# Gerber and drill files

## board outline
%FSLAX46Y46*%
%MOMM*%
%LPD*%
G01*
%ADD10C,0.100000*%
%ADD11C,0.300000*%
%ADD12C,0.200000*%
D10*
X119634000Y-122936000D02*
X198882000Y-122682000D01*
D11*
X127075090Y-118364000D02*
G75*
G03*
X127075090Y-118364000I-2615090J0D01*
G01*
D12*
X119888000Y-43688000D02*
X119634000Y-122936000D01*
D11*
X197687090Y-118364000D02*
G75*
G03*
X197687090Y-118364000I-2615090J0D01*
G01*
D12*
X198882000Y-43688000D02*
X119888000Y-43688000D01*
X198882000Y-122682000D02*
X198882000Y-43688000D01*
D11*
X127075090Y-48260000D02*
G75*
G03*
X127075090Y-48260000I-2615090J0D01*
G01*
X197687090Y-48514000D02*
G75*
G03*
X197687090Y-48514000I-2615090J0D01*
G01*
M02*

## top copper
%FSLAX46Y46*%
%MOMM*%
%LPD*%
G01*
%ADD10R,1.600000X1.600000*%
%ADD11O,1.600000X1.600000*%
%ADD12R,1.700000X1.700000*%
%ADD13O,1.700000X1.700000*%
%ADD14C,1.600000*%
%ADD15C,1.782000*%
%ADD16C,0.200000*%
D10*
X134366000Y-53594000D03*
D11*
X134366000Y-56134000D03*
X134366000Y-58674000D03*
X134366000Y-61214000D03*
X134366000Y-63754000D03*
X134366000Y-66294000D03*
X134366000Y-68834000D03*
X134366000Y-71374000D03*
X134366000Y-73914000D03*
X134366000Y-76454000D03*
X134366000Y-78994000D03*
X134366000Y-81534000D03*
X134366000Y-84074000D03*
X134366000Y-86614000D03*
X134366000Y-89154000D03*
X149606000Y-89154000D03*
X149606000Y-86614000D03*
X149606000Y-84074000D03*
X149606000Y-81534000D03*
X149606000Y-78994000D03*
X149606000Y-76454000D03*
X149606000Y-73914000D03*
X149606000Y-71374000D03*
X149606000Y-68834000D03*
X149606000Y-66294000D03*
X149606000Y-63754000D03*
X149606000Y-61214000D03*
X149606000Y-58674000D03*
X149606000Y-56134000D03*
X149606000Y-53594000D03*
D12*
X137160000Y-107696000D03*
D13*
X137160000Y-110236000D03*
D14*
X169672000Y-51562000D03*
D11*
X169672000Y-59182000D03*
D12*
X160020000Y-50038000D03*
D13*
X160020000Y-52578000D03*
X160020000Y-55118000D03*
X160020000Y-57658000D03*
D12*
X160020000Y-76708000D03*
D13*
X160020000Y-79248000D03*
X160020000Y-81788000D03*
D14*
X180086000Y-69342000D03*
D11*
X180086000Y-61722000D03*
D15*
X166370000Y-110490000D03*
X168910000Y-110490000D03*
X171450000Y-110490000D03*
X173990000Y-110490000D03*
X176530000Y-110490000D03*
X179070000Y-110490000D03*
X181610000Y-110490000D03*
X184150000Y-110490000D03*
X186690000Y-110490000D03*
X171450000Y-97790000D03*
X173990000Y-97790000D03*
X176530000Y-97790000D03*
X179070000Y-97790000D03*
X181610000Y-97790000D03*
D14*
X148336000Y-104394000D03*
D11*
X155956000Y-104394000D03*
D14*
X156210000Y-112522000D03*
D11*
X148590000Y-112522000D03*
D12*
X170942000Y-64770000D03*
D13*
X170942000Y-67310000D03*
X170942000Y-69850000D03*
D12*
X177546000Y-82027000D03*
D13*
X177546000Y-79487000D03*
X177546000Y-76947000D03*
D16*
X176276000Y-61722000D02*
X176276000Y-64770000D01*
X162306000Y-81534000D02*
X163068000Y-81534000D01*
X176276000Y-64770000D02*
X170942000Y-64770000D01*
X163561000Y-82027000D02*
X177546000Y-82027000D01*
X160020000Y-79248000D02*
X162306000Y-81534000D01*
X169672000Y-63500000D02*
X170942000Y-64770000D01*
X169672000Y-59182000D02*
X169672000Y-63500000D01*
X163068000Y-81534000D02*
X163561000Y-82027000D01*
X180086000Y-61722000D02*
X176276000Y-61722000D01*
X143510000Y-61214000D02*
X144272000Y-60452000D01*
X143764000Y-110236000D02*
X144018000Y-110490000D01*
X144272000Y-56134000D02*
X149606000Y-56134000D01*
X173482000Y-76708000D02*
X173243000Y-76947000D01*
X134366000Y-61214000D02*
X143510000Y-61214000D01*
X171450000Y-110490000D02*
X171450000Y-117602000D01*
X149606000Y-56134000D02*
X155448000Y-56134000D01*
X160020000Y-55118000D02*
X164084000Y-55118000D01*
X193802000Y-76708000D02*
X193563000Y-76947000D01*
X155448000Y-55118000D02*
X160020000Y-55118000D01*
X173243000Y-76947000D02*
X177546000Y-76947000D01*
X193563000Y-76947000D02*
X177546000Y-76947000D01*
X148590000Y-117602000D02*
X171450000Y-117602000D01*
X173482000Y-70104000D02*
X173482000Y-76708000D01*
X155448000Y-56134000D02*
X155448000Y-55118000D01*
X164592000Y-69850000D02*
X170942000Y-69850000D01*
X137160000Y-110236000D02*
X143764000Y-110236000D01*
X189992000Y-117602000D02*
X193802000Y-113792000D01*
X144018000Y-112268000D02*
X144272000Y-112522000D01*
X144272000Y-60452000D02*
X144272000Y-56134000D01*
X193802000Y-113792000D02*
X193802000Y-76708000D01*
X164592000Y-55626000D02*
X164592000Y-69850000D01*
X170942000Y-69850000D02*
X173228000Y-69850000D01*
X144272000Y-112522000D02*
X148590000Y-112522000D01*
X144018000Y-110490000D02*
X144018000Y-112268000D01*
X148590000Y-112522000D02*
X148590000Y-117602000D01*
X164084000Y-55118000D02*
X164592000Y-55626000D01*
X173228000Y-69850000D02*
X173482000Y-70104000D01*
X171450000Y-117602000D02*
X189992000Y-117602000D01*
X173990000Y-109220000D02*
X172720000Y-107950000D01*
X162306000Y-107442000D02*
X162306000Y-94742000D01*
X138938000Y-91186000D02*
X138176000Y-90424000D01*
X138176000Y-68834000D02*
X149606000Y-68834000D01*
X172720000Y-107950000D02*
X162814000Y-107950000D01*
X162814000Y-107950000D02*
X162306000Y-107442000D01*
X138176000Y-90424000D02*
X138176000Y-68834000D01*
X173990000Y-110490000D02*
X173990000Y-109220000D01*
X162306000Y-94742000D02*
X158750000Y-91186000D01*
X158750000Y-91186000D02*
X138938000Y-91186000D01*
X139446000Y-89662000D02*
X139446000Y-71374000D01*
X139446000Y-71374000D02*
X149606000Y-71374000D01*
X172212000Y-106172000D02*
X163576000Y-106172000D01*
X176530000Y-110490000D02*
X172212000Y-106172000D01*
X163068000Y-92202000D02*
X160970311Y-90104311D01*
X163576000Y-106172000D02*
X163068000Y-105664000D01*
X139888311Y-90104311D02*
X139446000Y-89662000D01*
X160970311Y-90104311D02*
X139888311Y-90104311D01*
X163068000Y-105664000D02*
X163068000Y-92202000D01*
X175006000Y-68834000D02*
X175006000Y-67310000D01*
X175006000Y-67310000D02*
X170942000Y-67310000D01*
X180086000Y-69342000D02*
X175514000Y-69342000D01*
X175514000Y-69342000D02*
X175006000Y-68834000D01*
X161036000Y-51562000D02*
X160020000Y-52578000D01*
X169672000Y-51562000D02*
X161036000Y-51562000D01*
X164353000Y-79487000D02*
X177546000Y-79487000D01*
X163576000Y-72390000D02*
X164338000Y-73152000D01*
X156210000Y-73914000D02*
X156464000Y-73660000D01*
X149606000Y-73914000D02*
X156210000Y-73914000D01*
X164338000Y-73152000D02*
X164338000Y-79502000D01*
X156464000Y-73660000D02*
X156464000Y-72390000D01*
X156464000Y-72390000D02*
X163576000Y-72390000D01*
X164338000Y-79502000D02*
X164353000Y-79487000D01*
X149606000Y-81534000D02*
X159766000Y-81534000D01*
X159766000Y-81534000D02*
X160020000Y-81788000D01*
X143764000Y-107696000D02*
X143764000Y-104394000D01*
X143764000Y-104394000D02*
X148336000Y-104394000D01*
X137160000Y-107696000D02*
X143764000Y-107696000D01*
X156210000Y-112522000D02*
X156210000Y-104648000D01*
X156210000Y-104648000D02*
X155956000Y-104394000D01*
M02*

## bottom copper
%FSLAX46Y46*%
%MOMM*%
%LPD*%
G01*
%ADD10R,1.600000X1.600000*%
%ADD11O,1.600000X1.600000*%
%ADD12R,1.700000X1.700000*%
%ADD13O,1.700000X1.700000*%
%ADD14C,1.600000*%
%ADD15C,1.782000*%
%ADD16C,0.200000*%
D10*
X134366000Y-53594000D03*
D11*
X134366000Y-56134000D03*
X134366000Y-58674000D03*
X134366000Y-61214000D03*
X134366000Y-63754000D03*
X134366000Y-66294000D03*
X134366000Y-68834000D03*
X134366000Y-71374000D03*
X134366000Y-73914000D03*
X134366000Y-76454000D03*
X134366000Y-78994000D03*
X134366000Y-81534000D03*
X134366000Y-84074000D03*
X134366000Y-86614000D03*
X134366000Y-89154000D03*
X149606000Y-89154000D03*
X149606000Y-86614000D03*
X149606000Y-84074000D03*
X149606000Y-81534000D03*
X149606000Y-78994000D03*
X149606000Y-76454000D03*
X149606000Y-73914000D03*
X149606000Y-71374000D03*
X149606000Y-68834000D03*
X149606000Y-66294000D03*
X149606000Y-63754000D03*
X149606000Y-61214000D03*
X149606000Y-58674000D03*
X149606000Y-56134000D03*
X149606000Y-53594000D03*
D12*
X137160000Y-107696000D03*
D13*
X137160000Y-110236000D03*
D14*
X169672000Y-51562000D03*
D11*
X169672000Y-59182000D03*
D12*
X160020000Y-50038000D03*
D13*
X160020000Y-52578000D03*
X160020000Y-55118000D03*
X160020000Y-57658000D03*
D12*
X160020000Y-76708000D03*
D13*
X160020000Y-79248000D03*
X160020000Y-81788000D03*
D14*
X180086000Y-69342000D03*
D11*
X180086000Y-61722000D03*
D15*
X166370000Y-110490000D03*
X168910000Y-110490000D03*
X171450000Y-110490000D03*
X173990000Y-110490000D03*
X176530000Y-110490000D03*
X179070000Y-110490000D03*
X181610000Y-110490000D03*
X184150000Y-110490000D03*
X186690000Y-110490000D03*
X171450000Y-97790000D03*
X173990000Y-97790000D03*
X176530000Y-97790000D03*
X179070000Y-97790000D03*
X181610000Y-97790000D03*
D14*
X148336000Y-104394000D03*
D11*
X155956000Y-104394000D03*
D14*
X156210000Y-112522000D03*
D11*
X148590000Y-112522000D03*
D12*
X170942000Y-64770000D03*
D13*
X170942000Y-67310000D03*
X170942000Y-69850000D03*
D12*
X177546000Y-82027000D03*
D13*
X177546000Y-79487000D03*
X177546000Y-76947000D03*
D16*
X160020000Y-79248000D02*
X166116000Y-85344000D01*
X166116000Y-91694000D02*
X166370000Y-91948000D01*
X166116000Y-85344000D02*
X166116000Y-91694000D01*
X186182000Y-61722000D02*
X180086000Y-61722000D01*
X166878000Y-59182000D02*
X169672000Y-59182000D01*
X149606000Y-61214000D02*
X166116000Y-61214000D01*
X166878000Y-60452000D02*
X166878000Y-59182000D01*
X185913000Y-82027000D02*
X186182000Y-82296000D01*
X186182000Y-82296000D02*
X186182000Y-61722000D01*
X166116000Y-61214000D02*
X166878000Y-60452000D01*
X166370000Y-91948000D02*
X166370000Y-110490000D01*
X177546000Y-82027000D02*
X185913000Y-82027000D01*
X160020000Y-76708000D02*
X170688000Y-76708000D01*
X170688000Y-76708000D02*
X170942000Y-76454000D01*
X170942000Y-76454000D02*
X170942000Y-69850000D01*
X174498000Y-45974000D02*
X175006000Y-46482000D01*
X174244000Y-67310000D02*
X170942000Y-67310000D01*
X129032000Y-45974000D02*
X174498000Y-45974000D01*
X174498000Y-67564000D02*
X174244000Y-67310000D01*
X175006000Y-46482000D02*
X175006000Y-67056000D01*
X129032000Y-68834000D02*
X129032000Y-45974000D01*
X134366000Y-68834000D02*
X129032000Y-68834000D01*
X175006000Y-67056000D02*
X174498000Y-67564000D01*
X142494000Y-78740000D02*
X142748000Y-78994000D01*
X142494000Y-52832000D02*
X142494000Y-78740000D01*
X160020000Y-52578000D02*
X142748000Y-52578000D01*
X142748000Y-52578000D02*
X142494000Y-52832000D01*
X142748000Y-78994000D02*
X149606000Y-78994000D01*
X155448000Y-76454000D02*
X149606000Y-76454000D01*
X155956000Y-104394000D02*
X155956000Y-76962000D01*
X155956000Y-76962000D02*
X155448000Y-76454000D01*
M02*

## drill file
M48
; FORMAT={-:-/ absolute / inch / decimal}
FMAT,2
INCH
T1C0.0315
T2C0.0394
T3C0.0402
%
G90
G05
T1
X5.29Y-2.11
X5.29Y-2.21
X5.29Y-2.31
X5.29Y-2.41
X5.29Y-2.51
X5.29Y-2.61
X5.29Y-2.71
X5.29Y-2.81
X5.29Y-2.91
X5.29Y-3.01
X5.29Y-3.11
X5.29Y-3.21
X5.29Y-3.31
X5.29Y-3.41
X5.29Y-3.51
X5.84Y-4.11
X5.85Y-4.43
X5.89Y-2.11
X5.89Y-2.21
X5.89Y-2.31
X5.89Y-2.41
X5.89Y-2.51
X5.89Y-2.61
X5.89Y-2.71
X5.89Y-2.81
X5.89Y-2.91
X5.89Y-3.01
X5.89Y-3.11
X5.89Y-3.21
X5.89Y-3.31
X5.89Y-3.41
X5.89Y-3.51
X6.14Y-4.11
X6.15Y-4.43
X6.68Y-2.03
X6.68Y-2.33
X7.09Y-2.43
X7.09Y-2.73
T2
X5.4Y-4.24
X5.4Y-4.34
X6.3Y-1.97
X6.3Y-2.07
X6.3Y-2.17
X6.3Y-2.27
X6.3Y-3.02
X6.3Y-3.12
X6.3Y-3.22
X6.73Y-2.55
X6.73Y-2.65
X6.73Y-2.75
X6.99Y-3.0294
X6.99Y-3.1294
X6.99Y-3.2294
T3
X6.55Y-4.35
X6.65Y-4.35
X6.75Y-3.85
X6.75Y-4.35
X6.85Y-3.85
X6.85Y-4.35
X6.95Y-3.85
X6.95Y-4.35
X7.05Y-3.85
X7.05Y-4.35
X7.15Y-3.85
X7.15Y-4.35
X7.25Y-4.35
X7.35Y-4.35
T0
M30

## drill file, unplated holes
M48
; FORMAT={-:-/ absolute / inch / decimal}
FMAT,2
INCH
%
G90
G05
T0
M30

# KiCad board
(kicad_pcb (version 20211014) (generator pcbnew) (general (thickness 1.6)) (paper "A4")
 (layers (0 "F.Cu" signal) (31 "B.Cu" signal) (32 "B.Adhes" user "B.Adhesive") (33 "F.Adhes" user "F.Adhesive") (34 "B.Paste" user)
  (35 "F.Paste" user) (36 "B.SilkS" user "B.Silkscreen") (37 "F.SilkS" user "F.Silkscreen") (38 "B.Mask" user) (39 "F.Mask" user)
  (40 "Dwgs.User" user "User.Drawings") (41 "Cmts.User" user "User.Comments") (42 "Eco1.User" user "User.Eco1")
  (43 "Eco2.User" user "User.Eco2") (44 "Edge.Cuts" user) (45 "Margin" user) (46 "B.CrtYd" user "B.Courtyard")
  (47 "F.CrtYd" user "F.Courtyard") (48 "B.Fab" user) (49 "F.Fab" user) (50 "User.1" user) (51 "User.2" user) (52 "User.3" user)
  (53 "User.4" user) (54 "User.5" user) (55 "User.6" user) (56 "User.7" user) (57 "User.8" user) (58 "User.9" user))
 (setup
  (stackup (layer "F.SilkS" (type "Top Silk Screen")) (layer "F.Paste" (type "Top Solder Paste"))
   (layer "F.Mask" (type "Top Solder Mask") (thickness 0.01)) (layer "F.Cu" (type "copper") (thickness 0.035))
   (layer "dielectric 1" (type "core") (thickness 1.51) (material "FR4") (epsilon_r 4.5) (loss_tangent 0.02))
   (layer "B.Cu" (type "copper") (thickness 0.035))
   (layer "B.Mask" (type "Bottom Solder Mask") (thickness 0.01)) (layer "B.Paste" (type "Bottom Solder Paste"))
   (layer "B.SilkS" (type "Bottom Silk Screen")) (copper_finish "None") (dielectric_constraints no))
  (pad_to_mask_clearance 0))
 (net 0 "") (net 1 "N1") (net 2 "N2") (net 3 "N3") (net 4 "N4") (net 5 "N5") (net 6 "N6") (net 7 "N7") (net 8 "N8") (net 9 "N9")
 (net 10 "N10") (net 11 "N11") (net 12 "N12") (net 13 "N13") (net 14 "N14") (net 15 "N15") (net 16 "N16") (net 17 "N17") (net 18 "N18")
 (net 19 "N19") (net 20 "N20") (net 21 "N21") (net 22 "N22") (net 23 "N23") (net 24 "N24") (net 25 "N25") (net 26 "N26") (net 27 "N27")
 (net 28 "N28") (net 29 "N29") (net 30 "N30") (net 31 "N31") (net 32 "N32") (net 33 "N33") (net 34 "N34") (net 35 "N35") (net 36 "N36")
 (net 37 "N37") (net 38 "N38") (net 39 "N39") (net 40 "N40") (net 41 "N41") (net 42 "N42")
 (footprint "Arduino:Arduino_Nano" (layer "F.Cu") (at 134.366 53.594)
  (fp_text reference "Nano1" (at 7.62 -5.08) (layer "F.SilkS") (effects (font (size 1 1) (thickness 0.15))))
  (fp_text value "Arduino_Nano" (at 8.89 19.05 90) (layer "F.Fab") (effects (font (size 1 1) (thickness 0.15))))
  (pad "1" thru_hole rect locked (at 0 0) (size 1.6 1.6) (drill 0.8) (layers *.Cu *.Mask) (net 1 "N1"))
  (pad "2" thru_hole oval locked (at 0 2.54) (size 1.6 1.6) (drill 0.8) (layers *.Cu *.Mask) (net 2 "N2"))
  (pad "3" thru_hole oval locked (at 0 5.08) (size 1.6 1.6) (drill 0.8) (layers *.Cu *.Mask) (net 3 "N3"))
  (pad "4" thru_hole oval locked (at 0 7.62) (size 1.6 1.6) (drill 0.8) (layers *.Cu *.Mask) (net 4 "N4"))
  (pad "5" thru_hole oval locked (at 0 10.16) (size 1.6 1.6) (drill 0.8) (layers *.Cu *.Mask) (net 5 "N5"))
  (pad "6" thru_hole oval locked (at 0 12.7) (size 1.6 1.6) (drill 0.8) (layers *.Cu *.Mask) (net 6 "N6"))
  (pad "7" thru_hole oval locked (at 0 15.24) (size 1.6 1.6) (drill 0.8) (layers *.Cu *.Mask) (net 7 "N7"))
  (pad "8" thru_hole oval locked (at 0 17.78) (size 1.6 1.6) (drill 0.8) (layers *.Cu *.Mask) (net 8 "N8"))
  (pad "9" thru_hole oval locked (at 0 20.32) (size 1.6 1.6) (drill 0.8) (layers *.Cu *.Mask) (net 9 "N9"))
  (pad "10" thru_hole oval locked (at 0 22.86) (size 1.6 1.6) (drill 0.8) (layers *.Cu *.Mask) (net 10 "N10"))
  (pad "11" thru_hole oval locked (at 0 25.4) (size 1.6 1.6) (drill 0.8) (layers *.Cu *.Mask) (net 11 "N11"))
  (pad "12" thru_hole oval locked (at 0 27.94) (size 1.6 1.6) (drill 0.8) (layers *.Cu *.Mask) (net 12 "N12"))
  (pad "13" thru_hole oval locked (at 0 30.48) (size 1.6 1.6) (drill 0.8) (layers *.Cu *.Mask) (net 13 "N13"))
  (pad "14" thru_hole oval locked (at 0 33.02) (size 1.6 1.6) (drill 0.8) (layers *.Cu *.Mask) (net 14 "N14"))
  (pad "15" thru_hole oval locked (at 0 35.56) (size 1.6 1.6) (drill 0.8) (layers *.Cu *.Mask) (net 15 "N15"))
  (pad "16" thru_hole oval locked (at 15.24 35.56) (size 1.6 1.6) (drill 0.8) (layers *.Cu *.Mask) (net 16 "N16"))
  (pad "17" thru_hole oval locked (at 15.24 33.02) (size 1.6 1.6) (drill 0.8) (layers *.Cu *.Mask) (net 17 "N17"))
  (pad "18" thru_hole oval locked (at 15.24 30.48) (size 1.6 1.6) (drill 0.8) (layers *.Cu *.Mask) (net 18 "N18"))
  (pad "19" thru_hole oval locked (at 15.24 27.94) (size 1.6 1.6) (drill 0.8) (layers *.Cu *.Mask) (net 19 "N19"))
  (pad "20" thru_hole oval locked (at 15.24 25.4) (size 1.6 1.6) (drill 0.8) (layers *.Cu *.Mask) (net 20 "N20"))
  (pad "21" thru_hole oval locked (at 15.24 22.86) (size 1.6 1.6) (drill 0.8) (layers *.Cu *.Mask) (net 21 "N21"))
  (pad "22" thru_hole oval locked (at 15.24 20.32) (size 1.6 1.6) (drill 0.8) (layers *.Cu *.Mask) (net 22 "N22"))
  (pad "23" thru_hole oval locked (at 15.24 17.78) (size 1.6 1.6) (drill 0.8) (layers *.Cu *.Mask) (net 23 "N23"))
  (pad "24" thru_hole oval locked (at 15.24 15.24) (size 1.6 1.6) (drill 0.8) (layers *.Cu *.Mask) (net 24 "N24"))
  (pad "25" thru_hole oval locked (at 15.24 12.7) (size 1.6 1.6) (drill 0.8) (layers *.Cu *.Mask) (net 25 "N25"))
  (pad "26" thru_hole oval locked (at 15.24 10.16) (size 1.6 1.6) (drill 0.8) (layers *.Cu *.Mask) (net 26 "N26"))
  (pad "27" thru_hole oval locked (at 15.24 7.62) (size 1.6 1.6) (drill 0.8) (layers *.Cu *.Mask) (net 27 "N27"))
  (pad "28" thru_hole oval locked (at 15.24 5.08) (size 1.6 1.6) (drill 0.8) (layers *.Cu *.Mask) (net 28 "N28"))
  (pad "29" thru_hole oval locked (at 15.24 2.54) (size 1.6 1.6) (drill 0.8) (layers *.Cu *.Mask) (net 4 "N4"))
  (pad "30" thru_hole oval locked (at 15.24 0) (size 1.6 1.6) (drill 0.8) (layers *.Cu *.Mask) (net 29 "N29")))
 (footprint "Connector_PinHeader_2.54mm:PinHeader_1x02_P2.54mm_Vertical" (layer "F.Cu") (at 137.16 107.696)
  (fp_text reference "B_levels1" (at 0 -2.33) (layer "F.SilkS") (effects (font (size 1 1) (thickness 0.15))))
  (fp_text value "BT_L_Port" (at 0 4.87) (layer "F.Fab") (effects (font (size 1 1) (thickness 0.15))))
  (pad "1" thru_hole rect (at 0 0) (size 1.7 1.7) (drill 1) (layers *.Cu *.Mask) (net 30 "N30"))
  (pad "2" thru_hole oval (at 0 2.54) (size 1.7 1.7) (drill 1) (layers *.Cu *.Mask) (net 4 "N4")))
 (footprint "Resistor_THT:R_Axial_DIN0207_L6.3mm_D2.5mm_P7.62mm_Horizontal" (layer "F.Cu") (at 169.672 51.562 -90)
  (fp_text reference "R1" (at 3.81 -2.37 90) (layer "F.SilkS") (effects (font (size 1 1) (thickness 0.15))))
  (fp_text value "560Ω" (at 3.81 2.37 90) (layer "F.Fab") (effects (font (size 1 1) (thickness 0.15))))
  (pad "1" thru_hole circle (at 0 0 270) (size 1.6 1.6) (drill 0.8) (layers *.Cu *.Mask) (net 20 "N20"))
  (pad "2" thru_hole oval (at 7.62 0 270) (size 1.6 1.6) (drill 0.8) (layers *.Cu *.Mask) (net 27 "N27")))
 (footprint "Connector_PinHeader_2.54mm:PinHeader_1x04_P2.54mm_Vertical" (layer "F.Cu") (at 160.02 50.038)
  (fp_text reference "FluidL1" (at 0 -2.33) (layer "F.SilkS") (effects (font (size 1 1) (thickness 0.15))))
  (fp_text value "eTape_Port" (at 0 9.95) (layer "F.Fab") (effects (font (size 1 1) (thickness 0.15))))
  (pad "1" thru_hole rect (at 0 0) (size 1.7 1.7) (drill 1) (layers *.Cu *.Mask) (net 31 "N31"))
  (pad "2" thru_hole oval (at 0 2.54) (size 1.7 1.7) (drill 1) (layers *.Cu *.Mask) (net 20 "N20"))
  (pad "3" thru_hole oval (at 0 5.08) (size 1.7 1.7) (drill 1) (layers *.Cu *.Mask) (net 4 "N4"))
  (pad "4" thru_hole oval (at 0 7.62) (size 1.7 1.7) (drill 1) (layers *.Cu *.Mask) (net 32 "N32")))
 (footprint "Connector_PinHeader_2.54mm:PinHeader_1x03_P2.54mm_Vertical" (layer "F.Cu") (at 160.02 76.708)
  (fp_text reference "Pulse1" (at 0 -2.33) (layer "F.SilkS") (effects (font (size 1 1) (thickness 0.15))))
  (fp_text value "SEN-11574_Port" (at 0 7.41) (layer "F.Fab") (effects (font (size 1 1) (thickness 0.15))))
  (pad "1" thru_hole rect (at 0 0) (size 1.7 1.7) (drill 1) (layers *.Cu *.Mask) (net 4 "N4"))
  (pad "2" thru_hole oval (at 0 2.54) (size 1.7 1.7) (drill 1) (layers *.Cu *.Mask) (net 27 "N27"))
  (pad "3" thru_hole oval (at 0 5.08) (size 1.7 1.7) (drill 1) (layers *.Cu *.Mask) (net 19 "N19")))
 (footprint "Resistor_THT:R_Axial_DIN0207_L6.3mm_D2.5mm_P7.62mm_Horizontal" (layer "F.Cu") (at 180.086 69.342 90)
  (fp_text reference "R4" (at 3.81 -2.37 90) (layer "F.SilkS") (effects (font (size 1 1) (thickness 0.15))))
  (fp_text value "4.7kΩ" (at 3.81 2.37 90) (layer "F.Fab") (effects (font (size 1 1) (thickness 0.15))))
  (pad "1" thru_hole circle (at 0 0 90) (size 1.6 1.6) (drill 0.8) (layers *.Cu *.Mask) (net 7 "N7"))
  (pad "2" thru_hole oval (at 7.62 0 90) (size 1.6 1.6) (drill 0.8) (layers *.Cu *.Mask) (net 27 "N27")))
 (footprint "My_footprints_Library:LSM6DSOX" (layer "F.Cu") (at 176.53 104.14)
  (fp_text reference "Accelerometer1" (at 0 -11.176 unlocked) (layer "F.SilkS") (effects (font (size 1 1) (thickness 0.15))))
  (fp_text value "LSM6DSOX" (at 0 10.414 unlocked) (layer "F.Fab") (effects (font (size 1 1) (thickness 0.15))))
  (pad "1" thru_hole circle (at -10.16 6.35) (size 1.782 1.782) (drill 1.02) (layers *.Cu *.Mask) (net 27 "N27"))
  (pad "2" thru_hole circle (at -7.62 6.35) (size 1.782 1.782) (drill 1.02) (layers *.Cu *.Mask) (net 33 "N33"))
  (pad "3" thru_hole circle (at -5.08 6.35) (size 1.782 1.782) (drill 1.02) (layers *.Cu *.Mask) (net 4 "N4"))
  (pad "4" thru_hole circle (at -2.54 6.35) (size 1.782 1.782) (drill 1.02) (layers *.Cu *.Mask) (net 24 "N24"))
  (pad "5" thru_hole circle (at 0 6.35) (size 1.782 1.782) (drill 1.02) (layers *.Cu *.Mask) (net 23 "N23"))
  (pad "6" thru_hole circle (at 2.54 6.35) (size 1.782 1.782) (drill 1.02) (layers *.Cu *.Mask) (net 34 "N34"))
  (pad "7" thru_hole circle (at 5.08 6.35) (size 1.782 1.782) (drill 1.02) (layers *.Cu *.Mask) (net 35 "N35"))
  (pad "8" thru_hole circle (at 7.62 6.35) (size 1.782 1.782) (drill 1.02) (layers *.Cu *.Mask) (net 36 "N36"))
  (pad "9" thru_hole circle (at 10.16 6.35) (size 1.782 1.782) (drill 1.02) (layers *.Cu *.Mask) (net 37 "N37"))
  (pad "10" thru_hole circle (at -5.08 -6.35) (size 1.782 1.782) (drill 1.02) (layers *.Cu *.Mask) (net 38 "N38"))
  (pad "11" thru_hole circle (at -2.54 -6.35) (size 1.782 1.782) (drill 1.02) (layers *.Cu *.Mask) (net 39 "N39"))
  (pad "12" thru_hole circle (at 0 -6.35) (size 1.782 1.782) (drill 1.02) (layers *.Cu *.Mask) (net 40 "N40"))
  (pad "13" thru_hole circle (at 2.54 -6.35) (size 1.782 1.782) (drill 1.02) (layers *.Cu *.Mask) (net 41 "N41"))
  (pad "14" thru_hole circle (at 5.08 -6.35) (size 1.782 1.782) (drill 1.02) (layers *.Cu *.Mask) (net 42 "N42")))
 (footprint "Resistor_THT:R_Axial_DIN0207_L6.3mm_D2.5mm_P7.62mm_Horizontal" (layer "F.Cu") (at 148.336 104.394)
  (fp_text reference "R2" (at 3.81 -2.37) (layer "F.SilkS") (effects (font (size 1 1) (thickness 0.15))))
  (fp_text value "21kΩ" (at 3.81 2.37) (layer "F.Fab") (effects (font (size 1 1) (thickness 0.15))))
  (pad "1" thru_hole circle (at 0 0) (size 1.6 1.6) (drill 0.8) (layers *.Cu *.Mask) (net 30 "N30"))
  (pad "2" thru_hole oval (at 7.62 0) (size 1.6 1.6) (drill 0.8) (layers *.Cu *.Mask) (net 21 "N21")))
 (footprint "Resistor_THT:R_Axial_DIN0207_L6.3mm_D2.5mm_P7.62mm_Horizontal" (layer "F.Cu") (at 156.21 112.522 180)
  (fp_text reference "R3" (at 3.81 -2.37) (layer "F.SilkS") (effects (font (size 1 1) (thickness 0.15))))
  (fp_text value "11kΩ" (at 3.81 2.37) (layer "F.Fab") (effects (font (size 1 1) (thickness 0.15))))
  (pad "1" thru_hole circle (at 0 0 180) (size 1.6 1.6) (drill 0.8) (layers *.Cu *.Mask) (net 21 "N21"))
  (pad "2" thru_hole oval (at 7.62 0 180) (size 1.6 1.6) (drill 0.8) (layers *.Cu *.Mask) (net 4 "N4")))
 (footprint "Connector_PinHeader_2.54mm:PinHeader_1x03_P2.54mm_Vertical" (layer "F.Cu") (at 170.942 64.77)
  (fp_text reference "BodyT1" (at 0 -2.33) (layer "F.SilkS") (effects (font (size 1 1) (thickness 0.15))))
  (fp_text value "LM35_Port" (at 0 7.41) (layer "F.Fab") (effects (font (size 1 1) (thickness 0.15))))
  (pad "1" thru_hole rect (at 0 0) (size 1.7 1.7) (drill 1) (layers *.Cu *.Mask) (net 27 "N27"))
  (pad "2" thru_hole oval (at 0 2.54) (size 1.7 1.7) (drill 1) (layers *.Cu *.Mask) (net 7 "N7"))
  (pad "3" thru_hole oval (at 0 5.08) (size 1.7 1.7) (drill 1) (layers *.Cu *.Mask) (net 4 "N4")))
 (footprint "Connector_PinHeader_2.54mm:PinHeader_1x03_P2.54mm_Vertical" (layer "F.Cu") (at 177.546 82.027 180)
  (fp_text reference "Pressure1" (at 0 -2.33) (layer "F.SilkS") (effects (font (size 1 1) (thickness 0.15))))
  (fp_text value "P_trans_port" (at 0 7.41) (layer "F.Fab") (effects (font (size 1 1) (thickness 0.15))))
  (pad "1" thru_hole rect (at 0 0 180) (size 1.7 1.7) (drill 1) (layers *.Cu *.Mask) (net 27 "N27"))
  (pad "2" thru_hole oval (at 0 2.54 180) (size 1.7 1.7) (drill 1) (layers *.Cu *.Mask) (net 22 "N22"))
  (pad "3" thru_hole oval (at 0 5.08 180) (size 1.7 1.7) (drill 1) (layers *.Cu *.Mask) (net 4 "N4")))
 (gr_line (start 119.634 122.936) (end 198.882 122.682) (layer "Edge.Cuts") (width 0.1))
 (gr_circle (center 124.46 118.364) (end 127.07509 118.364) (layer "Edge.Cuts") (width 0.3) (fill none))
 (gr_line (start 119.888 43.688) (end 119.634 122.936) (layer "Edge.Cuts") (width 0.2))
 (gr_circle (center 195.072 118.364) (end 197.68709 118.364) (layer "Edge.Cuts") (width 0.3) (fill none))
 (gr_line (start 198.882 43.688) (end 119.888 43.688) (layer "Edge.Cuts") (width 0.2))
 (gr_line (start 198.882 122.682) (end 198.882 43.688) (layer "Edge.Cuts") (width 0.2))
 (gr_circle (center 124.46 48.26) (end 127.07509 48.26) (layer "Edge.Cuts") (width 0.3) (fill none))
 (gr_circle (center 195.072 48.514) (end 197.68709 48.514) (layer "Edge.Cuts") (width 0.3) (fill none))
 (segment (start 176.276 61.722) (end 176.276 64.77) (width 0.2) (layer "F.Cu") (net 27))
 (segment (start 162.306 81.534) (end 163.068 81.534) (width 0.2) (layer "F.Cu") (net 27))
 (segment (start 176.276 64.77) (end 170.942 64.77) (width 0.2) (layer "F.Cu") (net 27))
 (segment (start 163.561 82.027) (end 177.546 82.027) (width 0.2) (layer "F.Cu") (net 27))
 (segment (start 160.02 79.248) (end 162.306 81.534) (width 0.2) (layer "F.Cu") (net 27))
 (segment (start 169.672 63.5) (end 170.942 64.77) (width 0.2) (layer "F.Cu") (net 27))
 (segment (start 169.672 59.182) (end 169.672 63.5) (width 0.2) (layer "F.Cu") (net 27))
 (segment (start 163.068 81.534) (end 163.561 82.027) (width 0.2) (layer "F.Cu") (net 27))
 (segment (start 180.086 61.722) (end 176.276 61.722) (width 0.2) (layer "F.Cu") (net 27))
 (segment (start 160.02 79.248) (end 166.116 85.344) (width 0.2) (layer "B.Cu") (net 27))
 (segment (start 166.116 91.694) (end 166.37 91.948) (width 0.2) (layer "B.Cu") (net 27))
 (segment (start 166.116 85.344) (end 166.116 91.694) (width 0.2) (layer "B.Cu") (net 27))
 (segment (start 186.182 61.722) (end 180.086 61.722) (width 0.2) (layer "B.Cu") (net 27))
 (segment (start 166.878 59.182) (end 169.672 59.182) (width 0.2) (layer "B.Cu") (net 27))
 (segment (start 149.606 61.214) (end 166.116 61.214) (width 0.2) (layer "B.Cu") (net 27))
 (segment (start 166.878 60.452) (end 166.878 59.182) (width 0.2) (layer "B.Cu") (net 27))
 (segment (start 185.913 82.027) (end 186.182 82.296) (width 0.2) (layer "B.Cu") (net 27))
 (segment (start 186.182 82.296) (end 186.182 61.722) (width 0.2) (layer "B.Cu") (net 27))
 (segment (start 166.116 61.214) (end 166.878 60.452) (width 0.2) (layer "B.Cu") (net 27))
 (segment (start 166.37 91.948) (end 166.37 110.49) (width 0.2) (layer "B.Cu") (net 27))
 (segment (start 177.546 82.027) (end 185.913 82.027) (width 0.2) (layer "B.Cu") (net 27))
 (segment (start 143.51 61.214) (end 144.272 60.452) (width 0.2) (layer "F.Cu") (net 4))
 (segment (start 143.764 110.236) (end 144.018 110.49) (width 0.2) (layer "F.Cu") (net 4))
 (segment (start 144.272 56.134) (end 149.606 56.134) (width 0.2) (layer "F.Cu") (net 4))
 (segment (start 173.482 76.708) (end 173.243 76.947) (width 0.2) (layer "F.Cu") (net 4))
 (segment (start 134.366 61.214) (end 143.51 61.214) (width 0.2) (layer "F.Cu") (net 4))
 (segment (start 171.45 110.49) (end 171.45 117.602) (width 0.2) (layer "F.Cu") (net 4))
 (segment (start 149.606 56.134) (end 155.448 56.134) (width 0.2) (layer "F.Cu") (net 4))
 (segment (start 160.02 55.118) (end 164.084 55.118) (width 0.2) (layer "F.Cu") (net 4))
 (segment (start 193.802 76.708) (end 193.563 76.947) (width 0.2) (layer "F.Cu") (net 4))
 (segment (start 155.448 55.118) (end 160.02 55.118) (width 0.2) (layer "F.Cu") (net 4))
 (segment (start 173.243 76.947) (end 177.546 76.947) (width 0.2) (layer "F.Cu") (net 4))
 (segment (start 193.563 76.947) (end 177.546 76.947) (width 0.2) (layer "F.Cu") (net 4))
 (segment (start 148.59 117.602) (end 171.45 117.602) (width 0.2) (layer "F.Cu") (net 4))
 (segment (start 173.482 70.104) (end 173.482 76.708) (width 0.2) (layer "F.Cu") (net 4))
 (segment (start 155.448 56.134) (end 155.448 55.118) (width 0.2) (layer "F.Cu") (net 4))
 (segment (start 164.592 69.85) (end 170.942 69.85) (width 0.2) (layer "F.Cu") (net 4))
 (segment (start 137.16 110.236) (end 143.764 110.236) (width 0.2) (layer "F.Cu") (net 4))
 (segment (start 189.992 117.602) (end 193.802 113.792) (width 0.2) (layer "F.Cu") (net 4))
 (segment (start 144.018 112.268) (end 144.272 112.522) (width 0.2) (layer "F.Cu") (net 4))
 (segment (start 144.272 60.452) (end 144.272 56.134) (width 0.2) (layer "F.Cu") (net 4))
 (segment (start 193.802 113.792) (end 193.802 76.708) (width 0.2) (layer "F.Cu") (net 4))
 (segment (start 164.592 55.626) (end 164.592 69.85) (width 0.2) (layer "F.Cu") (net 4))
 (segment (start 170.942 69.85) (end 173.228 69.85) (width 0.2) (layer "F.Cu") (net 4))
 (segment (start 144.272 112.522) (end 148.59 112.522) (width 0.2) (layer "F.Cu") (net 4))
 (segment (start 144.018 110.49) (end 144.018 112.268) (width 0.2) (layer "F.Cu") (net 4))
 (segment (start 148.59 112.522) (end 148.59 117.602) (width 0.2) (layer "F.Cu") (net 4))
 (segment (start 164.084 55.118) (end 164.592 55.626) (width 0.2) (layer "F.Cu") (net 4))
 (segment (start 173.228 69.85) (end 173.482 70.104) (width 0.2) (layer "F.Cu") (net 4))
 (segment (start 171.45 117.602) (end 189.992 117.602) (width 0.2) (layer "F.Cu") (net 4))
 (segment (start 160.02 76.708) (end 170.688 76.708) (width 0.2) (layer "B.Cu") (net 4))
 (segment (start 170.688 76.708) (end 170.942 76.454) (width 0.2) (layer "B.Cu") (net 4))
 (segment (start 170.942 76.454) (end 170.942 69.85) (width 0.2) (layer "B.Cu") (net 4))
 (segment (start 173.99 109.22) (end 172.72 107.95) (width 0.2) (layer "F.Cu") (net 24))
 (segment (start 162.306 107.442) (end 162.306 94.742) (width 0.2) (layer "F.Cu") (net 24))
 (segment (start 138.938 91.186) (end 138.176 90.424) (width 0.2) (layer "F.Cu") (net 24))
 (segment (start 138.176 68.834) (end 149.606 68.834) (width 0.2) (layer "F.Cu") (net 24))
 (segment (start 172.72 107.95) (end 162.814 107.95) (width 0.2) (layer "F.Cu") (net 24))
 (segment (start 162.814 107.95) (end 162.306 107.442) (width 0.2) (layer "F.Cu") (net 24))
 (segment (start 138.176 90.424) (end 138.176 68.834) (width 0.2) (layer "F.Cu") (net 24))
 (segment (start 173.99 110.49) (end 173.99 109.22) (width 0.2) (layer "F.Cu") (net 24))
 (segment (start 162.306 94.742) (end 158.75 91.186) (width 0.2) (layer "F.Cu") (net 24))
 (segment (start 158.75 91.186) (end 138.938 91.186) (width 0.2) (layer "F.Cu") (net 24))
 (segment (start 139.446 89.662) (end 139.446 71.374) (width 0.2) (layer "F.Cu") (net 23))
 (segment (start 139.446 71.374) (end 149.606 71.374) (width 0.2) (layer "F.Cu") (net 23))
 (segment (start 172.212 106.172) (end 163.576 106.172) (width 0.2) (layer "F.Cu") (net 23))
 (segment (start 176.53 110.49) (end 172.212 106.172) (width 0.2) (layer "F.Cu") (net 23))
 (segment (start 163.068 92.202) (end 160.970311 90.104311) (width 0.2) (layer "F.Cu") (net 23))
 (segment (start 163.576 106.172) (end 163.068 105.664) (width 0.2) (layer "F.Cu") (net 23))
 (segment (start 139.888311 90.104311) (end 139.446 89.662) (width 0.2) (layer "F.Cu") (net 23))
 (segment (start 160.970311 90.104311) (end 139.888311 90.104311) (width 0.2) (layer "F.Cu") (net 23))
 (segment (start 163.068 105.664) (end 163.068 92.202) (width 0.2) (layer "F.Cu") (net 23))
 (segment (start 175.006 68.834) (end 175.006 67.31) (width 0.2) (layer "F.Cu") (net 7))
 (segment (start 175.006 67.31) (end 170.942 67.31) (width 0.2) (layer "F.Cu") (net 7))
 (segment (start 180.086 69.342) (end 175.514 69.342) (width 0.2) (layer "F.Cu") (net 7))
 (segment (start 175.514 69.342) (end 175.006 68.834) (width 0.2) (layer "F.Cu") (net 7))
 (segment (start 174.498 45.974) (end 175.006 46.482) (width 0.2) (layer "B.Cu") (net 7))
 (segment (start 174.244 67.31) (end 170.942 67.31) (width 0.2) (layer "B.Cu") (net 7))
 (segment (start 129.032 45.974) (end 174.498 45.974) (width 0.2) (layer "B.Cu") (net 7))
 (segment (start 174.498 67.564) (end 174.244 67.31) (width 0.2) (layer "B.Cu") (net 7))
 (segment (start 175.006 46.482) (end 175.006 67.056) (width 0.2) (layer "B.Cu") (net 7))
 (segment (start 129.032 68.834) (end 129.032 45.974) (width 0.2) (layer "B.Cu") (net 7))
 (segment (start 134.366 68.834) (end 129.032 68.834) (width 0.2) (layer "B.Cu") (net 7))
 (segment (start 175.006 67.056) (end 174.498 67.564) (width 0.2) (layer "B.Cu") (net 7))
 (segment (start 161.036 51.562) (end 160.02 52.578) (width 0.2) (layer "F.Cu") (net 20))
 (segment (start 169.672 51.562) (end 161.036 51.562) (width 0.2) (layer "F.Cu") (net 20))
 (segment (start 142.494 78.74) (end 142.748 78.994) (width 0.2) (layer "B.Cu") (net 20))
 (segment (start 142.494 52.832) (end 142.494 78.74) (width 0.2) (layer "B.Cu") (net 20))
 (segment (start 160.02 52.578) (end 142.748 52.578) (width 0.2) (layer "B.Cu") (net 20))
 (segment (start 142.748 52.578) (end 142.494 52.832) (width 0.2) (layer "B.Cu") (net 20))
 (segment (start 142.748 78.994) (end 149.606 78.994) (width 0.2) (layer "B.Cu") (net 20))
 (segment (start 164.353 79.487) (end 177.546 79.487) (width 0.2) (layer "F.Cu") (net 22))
 (segment (start 163.576 72.39) (end 164.338 73.152) (width 0.2) (layer "F.Cu") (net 22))
 (segment (start 156.21 73.914) (end 156.464 73.66) (width 0.2) (layer "F.Cu") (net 22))
 (segment (start 149.606 73.914) (end 156.21 73.914) (width 0.2) (layer "F.Cu") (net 22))
 (segment (start 164.338 73.152) (end 164.338 79.502) (width 0.2) (layer "F.Cu") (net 22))
 (segment (start 156.464 73.66) (end 156.464 72.39) (width 0.2) (layer "F.Cu") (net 22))
 (segment (start 156.464 72.39) (end 163.576 72.39) (width 0.2) (layer "F.Cu") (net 22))
 (segment (start 164.338 79.502) (end 164.353 79.487) (width 0.2) (layer "F.Cu") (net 22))
 (segment (start 149.606 81.534) (end 159.766 81.534) (width 0.2) (layer "F.Cu") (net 19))
 (segment (start 159.766 81.534) (end 160.02 81.788) (width 0.2) (layer "F.Cu") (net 19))
 (segment (start 143.764 107.696) (end 143.764 104.394) (width 0.2) (layer "F.Cu") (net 30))
 (segment (start 143.764 104.394) (end 148.336 104.394) (width 0.2) (layer "F.Cu") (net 30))
 (segment (start 137.16 107.696) (end 143.764 107.696) (width 0.2) (layer "F.Cu") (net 30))
 (segment (start 156.21 112.522) (end 156.21 104.648) (width 0.2) (layer "F.Cu") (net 21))
 (segment (start 156.21 104.648) (end 155.956 104.394) (width 0.2) (layer "F.Cu") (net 21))
 (segment (start 155.448 76.454) (end 149.606 76.454) (width 0.2) (layer "B.Cu") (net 21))
 (segment (start 155.956 104.394) (end 155.956 76.962) (width 0.2) (layer "B.Cu") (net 21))
 (segment (start 155.956 76.962) (end 155.448 76.454) (width 0.2) (layer "B.Cu") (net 21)))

